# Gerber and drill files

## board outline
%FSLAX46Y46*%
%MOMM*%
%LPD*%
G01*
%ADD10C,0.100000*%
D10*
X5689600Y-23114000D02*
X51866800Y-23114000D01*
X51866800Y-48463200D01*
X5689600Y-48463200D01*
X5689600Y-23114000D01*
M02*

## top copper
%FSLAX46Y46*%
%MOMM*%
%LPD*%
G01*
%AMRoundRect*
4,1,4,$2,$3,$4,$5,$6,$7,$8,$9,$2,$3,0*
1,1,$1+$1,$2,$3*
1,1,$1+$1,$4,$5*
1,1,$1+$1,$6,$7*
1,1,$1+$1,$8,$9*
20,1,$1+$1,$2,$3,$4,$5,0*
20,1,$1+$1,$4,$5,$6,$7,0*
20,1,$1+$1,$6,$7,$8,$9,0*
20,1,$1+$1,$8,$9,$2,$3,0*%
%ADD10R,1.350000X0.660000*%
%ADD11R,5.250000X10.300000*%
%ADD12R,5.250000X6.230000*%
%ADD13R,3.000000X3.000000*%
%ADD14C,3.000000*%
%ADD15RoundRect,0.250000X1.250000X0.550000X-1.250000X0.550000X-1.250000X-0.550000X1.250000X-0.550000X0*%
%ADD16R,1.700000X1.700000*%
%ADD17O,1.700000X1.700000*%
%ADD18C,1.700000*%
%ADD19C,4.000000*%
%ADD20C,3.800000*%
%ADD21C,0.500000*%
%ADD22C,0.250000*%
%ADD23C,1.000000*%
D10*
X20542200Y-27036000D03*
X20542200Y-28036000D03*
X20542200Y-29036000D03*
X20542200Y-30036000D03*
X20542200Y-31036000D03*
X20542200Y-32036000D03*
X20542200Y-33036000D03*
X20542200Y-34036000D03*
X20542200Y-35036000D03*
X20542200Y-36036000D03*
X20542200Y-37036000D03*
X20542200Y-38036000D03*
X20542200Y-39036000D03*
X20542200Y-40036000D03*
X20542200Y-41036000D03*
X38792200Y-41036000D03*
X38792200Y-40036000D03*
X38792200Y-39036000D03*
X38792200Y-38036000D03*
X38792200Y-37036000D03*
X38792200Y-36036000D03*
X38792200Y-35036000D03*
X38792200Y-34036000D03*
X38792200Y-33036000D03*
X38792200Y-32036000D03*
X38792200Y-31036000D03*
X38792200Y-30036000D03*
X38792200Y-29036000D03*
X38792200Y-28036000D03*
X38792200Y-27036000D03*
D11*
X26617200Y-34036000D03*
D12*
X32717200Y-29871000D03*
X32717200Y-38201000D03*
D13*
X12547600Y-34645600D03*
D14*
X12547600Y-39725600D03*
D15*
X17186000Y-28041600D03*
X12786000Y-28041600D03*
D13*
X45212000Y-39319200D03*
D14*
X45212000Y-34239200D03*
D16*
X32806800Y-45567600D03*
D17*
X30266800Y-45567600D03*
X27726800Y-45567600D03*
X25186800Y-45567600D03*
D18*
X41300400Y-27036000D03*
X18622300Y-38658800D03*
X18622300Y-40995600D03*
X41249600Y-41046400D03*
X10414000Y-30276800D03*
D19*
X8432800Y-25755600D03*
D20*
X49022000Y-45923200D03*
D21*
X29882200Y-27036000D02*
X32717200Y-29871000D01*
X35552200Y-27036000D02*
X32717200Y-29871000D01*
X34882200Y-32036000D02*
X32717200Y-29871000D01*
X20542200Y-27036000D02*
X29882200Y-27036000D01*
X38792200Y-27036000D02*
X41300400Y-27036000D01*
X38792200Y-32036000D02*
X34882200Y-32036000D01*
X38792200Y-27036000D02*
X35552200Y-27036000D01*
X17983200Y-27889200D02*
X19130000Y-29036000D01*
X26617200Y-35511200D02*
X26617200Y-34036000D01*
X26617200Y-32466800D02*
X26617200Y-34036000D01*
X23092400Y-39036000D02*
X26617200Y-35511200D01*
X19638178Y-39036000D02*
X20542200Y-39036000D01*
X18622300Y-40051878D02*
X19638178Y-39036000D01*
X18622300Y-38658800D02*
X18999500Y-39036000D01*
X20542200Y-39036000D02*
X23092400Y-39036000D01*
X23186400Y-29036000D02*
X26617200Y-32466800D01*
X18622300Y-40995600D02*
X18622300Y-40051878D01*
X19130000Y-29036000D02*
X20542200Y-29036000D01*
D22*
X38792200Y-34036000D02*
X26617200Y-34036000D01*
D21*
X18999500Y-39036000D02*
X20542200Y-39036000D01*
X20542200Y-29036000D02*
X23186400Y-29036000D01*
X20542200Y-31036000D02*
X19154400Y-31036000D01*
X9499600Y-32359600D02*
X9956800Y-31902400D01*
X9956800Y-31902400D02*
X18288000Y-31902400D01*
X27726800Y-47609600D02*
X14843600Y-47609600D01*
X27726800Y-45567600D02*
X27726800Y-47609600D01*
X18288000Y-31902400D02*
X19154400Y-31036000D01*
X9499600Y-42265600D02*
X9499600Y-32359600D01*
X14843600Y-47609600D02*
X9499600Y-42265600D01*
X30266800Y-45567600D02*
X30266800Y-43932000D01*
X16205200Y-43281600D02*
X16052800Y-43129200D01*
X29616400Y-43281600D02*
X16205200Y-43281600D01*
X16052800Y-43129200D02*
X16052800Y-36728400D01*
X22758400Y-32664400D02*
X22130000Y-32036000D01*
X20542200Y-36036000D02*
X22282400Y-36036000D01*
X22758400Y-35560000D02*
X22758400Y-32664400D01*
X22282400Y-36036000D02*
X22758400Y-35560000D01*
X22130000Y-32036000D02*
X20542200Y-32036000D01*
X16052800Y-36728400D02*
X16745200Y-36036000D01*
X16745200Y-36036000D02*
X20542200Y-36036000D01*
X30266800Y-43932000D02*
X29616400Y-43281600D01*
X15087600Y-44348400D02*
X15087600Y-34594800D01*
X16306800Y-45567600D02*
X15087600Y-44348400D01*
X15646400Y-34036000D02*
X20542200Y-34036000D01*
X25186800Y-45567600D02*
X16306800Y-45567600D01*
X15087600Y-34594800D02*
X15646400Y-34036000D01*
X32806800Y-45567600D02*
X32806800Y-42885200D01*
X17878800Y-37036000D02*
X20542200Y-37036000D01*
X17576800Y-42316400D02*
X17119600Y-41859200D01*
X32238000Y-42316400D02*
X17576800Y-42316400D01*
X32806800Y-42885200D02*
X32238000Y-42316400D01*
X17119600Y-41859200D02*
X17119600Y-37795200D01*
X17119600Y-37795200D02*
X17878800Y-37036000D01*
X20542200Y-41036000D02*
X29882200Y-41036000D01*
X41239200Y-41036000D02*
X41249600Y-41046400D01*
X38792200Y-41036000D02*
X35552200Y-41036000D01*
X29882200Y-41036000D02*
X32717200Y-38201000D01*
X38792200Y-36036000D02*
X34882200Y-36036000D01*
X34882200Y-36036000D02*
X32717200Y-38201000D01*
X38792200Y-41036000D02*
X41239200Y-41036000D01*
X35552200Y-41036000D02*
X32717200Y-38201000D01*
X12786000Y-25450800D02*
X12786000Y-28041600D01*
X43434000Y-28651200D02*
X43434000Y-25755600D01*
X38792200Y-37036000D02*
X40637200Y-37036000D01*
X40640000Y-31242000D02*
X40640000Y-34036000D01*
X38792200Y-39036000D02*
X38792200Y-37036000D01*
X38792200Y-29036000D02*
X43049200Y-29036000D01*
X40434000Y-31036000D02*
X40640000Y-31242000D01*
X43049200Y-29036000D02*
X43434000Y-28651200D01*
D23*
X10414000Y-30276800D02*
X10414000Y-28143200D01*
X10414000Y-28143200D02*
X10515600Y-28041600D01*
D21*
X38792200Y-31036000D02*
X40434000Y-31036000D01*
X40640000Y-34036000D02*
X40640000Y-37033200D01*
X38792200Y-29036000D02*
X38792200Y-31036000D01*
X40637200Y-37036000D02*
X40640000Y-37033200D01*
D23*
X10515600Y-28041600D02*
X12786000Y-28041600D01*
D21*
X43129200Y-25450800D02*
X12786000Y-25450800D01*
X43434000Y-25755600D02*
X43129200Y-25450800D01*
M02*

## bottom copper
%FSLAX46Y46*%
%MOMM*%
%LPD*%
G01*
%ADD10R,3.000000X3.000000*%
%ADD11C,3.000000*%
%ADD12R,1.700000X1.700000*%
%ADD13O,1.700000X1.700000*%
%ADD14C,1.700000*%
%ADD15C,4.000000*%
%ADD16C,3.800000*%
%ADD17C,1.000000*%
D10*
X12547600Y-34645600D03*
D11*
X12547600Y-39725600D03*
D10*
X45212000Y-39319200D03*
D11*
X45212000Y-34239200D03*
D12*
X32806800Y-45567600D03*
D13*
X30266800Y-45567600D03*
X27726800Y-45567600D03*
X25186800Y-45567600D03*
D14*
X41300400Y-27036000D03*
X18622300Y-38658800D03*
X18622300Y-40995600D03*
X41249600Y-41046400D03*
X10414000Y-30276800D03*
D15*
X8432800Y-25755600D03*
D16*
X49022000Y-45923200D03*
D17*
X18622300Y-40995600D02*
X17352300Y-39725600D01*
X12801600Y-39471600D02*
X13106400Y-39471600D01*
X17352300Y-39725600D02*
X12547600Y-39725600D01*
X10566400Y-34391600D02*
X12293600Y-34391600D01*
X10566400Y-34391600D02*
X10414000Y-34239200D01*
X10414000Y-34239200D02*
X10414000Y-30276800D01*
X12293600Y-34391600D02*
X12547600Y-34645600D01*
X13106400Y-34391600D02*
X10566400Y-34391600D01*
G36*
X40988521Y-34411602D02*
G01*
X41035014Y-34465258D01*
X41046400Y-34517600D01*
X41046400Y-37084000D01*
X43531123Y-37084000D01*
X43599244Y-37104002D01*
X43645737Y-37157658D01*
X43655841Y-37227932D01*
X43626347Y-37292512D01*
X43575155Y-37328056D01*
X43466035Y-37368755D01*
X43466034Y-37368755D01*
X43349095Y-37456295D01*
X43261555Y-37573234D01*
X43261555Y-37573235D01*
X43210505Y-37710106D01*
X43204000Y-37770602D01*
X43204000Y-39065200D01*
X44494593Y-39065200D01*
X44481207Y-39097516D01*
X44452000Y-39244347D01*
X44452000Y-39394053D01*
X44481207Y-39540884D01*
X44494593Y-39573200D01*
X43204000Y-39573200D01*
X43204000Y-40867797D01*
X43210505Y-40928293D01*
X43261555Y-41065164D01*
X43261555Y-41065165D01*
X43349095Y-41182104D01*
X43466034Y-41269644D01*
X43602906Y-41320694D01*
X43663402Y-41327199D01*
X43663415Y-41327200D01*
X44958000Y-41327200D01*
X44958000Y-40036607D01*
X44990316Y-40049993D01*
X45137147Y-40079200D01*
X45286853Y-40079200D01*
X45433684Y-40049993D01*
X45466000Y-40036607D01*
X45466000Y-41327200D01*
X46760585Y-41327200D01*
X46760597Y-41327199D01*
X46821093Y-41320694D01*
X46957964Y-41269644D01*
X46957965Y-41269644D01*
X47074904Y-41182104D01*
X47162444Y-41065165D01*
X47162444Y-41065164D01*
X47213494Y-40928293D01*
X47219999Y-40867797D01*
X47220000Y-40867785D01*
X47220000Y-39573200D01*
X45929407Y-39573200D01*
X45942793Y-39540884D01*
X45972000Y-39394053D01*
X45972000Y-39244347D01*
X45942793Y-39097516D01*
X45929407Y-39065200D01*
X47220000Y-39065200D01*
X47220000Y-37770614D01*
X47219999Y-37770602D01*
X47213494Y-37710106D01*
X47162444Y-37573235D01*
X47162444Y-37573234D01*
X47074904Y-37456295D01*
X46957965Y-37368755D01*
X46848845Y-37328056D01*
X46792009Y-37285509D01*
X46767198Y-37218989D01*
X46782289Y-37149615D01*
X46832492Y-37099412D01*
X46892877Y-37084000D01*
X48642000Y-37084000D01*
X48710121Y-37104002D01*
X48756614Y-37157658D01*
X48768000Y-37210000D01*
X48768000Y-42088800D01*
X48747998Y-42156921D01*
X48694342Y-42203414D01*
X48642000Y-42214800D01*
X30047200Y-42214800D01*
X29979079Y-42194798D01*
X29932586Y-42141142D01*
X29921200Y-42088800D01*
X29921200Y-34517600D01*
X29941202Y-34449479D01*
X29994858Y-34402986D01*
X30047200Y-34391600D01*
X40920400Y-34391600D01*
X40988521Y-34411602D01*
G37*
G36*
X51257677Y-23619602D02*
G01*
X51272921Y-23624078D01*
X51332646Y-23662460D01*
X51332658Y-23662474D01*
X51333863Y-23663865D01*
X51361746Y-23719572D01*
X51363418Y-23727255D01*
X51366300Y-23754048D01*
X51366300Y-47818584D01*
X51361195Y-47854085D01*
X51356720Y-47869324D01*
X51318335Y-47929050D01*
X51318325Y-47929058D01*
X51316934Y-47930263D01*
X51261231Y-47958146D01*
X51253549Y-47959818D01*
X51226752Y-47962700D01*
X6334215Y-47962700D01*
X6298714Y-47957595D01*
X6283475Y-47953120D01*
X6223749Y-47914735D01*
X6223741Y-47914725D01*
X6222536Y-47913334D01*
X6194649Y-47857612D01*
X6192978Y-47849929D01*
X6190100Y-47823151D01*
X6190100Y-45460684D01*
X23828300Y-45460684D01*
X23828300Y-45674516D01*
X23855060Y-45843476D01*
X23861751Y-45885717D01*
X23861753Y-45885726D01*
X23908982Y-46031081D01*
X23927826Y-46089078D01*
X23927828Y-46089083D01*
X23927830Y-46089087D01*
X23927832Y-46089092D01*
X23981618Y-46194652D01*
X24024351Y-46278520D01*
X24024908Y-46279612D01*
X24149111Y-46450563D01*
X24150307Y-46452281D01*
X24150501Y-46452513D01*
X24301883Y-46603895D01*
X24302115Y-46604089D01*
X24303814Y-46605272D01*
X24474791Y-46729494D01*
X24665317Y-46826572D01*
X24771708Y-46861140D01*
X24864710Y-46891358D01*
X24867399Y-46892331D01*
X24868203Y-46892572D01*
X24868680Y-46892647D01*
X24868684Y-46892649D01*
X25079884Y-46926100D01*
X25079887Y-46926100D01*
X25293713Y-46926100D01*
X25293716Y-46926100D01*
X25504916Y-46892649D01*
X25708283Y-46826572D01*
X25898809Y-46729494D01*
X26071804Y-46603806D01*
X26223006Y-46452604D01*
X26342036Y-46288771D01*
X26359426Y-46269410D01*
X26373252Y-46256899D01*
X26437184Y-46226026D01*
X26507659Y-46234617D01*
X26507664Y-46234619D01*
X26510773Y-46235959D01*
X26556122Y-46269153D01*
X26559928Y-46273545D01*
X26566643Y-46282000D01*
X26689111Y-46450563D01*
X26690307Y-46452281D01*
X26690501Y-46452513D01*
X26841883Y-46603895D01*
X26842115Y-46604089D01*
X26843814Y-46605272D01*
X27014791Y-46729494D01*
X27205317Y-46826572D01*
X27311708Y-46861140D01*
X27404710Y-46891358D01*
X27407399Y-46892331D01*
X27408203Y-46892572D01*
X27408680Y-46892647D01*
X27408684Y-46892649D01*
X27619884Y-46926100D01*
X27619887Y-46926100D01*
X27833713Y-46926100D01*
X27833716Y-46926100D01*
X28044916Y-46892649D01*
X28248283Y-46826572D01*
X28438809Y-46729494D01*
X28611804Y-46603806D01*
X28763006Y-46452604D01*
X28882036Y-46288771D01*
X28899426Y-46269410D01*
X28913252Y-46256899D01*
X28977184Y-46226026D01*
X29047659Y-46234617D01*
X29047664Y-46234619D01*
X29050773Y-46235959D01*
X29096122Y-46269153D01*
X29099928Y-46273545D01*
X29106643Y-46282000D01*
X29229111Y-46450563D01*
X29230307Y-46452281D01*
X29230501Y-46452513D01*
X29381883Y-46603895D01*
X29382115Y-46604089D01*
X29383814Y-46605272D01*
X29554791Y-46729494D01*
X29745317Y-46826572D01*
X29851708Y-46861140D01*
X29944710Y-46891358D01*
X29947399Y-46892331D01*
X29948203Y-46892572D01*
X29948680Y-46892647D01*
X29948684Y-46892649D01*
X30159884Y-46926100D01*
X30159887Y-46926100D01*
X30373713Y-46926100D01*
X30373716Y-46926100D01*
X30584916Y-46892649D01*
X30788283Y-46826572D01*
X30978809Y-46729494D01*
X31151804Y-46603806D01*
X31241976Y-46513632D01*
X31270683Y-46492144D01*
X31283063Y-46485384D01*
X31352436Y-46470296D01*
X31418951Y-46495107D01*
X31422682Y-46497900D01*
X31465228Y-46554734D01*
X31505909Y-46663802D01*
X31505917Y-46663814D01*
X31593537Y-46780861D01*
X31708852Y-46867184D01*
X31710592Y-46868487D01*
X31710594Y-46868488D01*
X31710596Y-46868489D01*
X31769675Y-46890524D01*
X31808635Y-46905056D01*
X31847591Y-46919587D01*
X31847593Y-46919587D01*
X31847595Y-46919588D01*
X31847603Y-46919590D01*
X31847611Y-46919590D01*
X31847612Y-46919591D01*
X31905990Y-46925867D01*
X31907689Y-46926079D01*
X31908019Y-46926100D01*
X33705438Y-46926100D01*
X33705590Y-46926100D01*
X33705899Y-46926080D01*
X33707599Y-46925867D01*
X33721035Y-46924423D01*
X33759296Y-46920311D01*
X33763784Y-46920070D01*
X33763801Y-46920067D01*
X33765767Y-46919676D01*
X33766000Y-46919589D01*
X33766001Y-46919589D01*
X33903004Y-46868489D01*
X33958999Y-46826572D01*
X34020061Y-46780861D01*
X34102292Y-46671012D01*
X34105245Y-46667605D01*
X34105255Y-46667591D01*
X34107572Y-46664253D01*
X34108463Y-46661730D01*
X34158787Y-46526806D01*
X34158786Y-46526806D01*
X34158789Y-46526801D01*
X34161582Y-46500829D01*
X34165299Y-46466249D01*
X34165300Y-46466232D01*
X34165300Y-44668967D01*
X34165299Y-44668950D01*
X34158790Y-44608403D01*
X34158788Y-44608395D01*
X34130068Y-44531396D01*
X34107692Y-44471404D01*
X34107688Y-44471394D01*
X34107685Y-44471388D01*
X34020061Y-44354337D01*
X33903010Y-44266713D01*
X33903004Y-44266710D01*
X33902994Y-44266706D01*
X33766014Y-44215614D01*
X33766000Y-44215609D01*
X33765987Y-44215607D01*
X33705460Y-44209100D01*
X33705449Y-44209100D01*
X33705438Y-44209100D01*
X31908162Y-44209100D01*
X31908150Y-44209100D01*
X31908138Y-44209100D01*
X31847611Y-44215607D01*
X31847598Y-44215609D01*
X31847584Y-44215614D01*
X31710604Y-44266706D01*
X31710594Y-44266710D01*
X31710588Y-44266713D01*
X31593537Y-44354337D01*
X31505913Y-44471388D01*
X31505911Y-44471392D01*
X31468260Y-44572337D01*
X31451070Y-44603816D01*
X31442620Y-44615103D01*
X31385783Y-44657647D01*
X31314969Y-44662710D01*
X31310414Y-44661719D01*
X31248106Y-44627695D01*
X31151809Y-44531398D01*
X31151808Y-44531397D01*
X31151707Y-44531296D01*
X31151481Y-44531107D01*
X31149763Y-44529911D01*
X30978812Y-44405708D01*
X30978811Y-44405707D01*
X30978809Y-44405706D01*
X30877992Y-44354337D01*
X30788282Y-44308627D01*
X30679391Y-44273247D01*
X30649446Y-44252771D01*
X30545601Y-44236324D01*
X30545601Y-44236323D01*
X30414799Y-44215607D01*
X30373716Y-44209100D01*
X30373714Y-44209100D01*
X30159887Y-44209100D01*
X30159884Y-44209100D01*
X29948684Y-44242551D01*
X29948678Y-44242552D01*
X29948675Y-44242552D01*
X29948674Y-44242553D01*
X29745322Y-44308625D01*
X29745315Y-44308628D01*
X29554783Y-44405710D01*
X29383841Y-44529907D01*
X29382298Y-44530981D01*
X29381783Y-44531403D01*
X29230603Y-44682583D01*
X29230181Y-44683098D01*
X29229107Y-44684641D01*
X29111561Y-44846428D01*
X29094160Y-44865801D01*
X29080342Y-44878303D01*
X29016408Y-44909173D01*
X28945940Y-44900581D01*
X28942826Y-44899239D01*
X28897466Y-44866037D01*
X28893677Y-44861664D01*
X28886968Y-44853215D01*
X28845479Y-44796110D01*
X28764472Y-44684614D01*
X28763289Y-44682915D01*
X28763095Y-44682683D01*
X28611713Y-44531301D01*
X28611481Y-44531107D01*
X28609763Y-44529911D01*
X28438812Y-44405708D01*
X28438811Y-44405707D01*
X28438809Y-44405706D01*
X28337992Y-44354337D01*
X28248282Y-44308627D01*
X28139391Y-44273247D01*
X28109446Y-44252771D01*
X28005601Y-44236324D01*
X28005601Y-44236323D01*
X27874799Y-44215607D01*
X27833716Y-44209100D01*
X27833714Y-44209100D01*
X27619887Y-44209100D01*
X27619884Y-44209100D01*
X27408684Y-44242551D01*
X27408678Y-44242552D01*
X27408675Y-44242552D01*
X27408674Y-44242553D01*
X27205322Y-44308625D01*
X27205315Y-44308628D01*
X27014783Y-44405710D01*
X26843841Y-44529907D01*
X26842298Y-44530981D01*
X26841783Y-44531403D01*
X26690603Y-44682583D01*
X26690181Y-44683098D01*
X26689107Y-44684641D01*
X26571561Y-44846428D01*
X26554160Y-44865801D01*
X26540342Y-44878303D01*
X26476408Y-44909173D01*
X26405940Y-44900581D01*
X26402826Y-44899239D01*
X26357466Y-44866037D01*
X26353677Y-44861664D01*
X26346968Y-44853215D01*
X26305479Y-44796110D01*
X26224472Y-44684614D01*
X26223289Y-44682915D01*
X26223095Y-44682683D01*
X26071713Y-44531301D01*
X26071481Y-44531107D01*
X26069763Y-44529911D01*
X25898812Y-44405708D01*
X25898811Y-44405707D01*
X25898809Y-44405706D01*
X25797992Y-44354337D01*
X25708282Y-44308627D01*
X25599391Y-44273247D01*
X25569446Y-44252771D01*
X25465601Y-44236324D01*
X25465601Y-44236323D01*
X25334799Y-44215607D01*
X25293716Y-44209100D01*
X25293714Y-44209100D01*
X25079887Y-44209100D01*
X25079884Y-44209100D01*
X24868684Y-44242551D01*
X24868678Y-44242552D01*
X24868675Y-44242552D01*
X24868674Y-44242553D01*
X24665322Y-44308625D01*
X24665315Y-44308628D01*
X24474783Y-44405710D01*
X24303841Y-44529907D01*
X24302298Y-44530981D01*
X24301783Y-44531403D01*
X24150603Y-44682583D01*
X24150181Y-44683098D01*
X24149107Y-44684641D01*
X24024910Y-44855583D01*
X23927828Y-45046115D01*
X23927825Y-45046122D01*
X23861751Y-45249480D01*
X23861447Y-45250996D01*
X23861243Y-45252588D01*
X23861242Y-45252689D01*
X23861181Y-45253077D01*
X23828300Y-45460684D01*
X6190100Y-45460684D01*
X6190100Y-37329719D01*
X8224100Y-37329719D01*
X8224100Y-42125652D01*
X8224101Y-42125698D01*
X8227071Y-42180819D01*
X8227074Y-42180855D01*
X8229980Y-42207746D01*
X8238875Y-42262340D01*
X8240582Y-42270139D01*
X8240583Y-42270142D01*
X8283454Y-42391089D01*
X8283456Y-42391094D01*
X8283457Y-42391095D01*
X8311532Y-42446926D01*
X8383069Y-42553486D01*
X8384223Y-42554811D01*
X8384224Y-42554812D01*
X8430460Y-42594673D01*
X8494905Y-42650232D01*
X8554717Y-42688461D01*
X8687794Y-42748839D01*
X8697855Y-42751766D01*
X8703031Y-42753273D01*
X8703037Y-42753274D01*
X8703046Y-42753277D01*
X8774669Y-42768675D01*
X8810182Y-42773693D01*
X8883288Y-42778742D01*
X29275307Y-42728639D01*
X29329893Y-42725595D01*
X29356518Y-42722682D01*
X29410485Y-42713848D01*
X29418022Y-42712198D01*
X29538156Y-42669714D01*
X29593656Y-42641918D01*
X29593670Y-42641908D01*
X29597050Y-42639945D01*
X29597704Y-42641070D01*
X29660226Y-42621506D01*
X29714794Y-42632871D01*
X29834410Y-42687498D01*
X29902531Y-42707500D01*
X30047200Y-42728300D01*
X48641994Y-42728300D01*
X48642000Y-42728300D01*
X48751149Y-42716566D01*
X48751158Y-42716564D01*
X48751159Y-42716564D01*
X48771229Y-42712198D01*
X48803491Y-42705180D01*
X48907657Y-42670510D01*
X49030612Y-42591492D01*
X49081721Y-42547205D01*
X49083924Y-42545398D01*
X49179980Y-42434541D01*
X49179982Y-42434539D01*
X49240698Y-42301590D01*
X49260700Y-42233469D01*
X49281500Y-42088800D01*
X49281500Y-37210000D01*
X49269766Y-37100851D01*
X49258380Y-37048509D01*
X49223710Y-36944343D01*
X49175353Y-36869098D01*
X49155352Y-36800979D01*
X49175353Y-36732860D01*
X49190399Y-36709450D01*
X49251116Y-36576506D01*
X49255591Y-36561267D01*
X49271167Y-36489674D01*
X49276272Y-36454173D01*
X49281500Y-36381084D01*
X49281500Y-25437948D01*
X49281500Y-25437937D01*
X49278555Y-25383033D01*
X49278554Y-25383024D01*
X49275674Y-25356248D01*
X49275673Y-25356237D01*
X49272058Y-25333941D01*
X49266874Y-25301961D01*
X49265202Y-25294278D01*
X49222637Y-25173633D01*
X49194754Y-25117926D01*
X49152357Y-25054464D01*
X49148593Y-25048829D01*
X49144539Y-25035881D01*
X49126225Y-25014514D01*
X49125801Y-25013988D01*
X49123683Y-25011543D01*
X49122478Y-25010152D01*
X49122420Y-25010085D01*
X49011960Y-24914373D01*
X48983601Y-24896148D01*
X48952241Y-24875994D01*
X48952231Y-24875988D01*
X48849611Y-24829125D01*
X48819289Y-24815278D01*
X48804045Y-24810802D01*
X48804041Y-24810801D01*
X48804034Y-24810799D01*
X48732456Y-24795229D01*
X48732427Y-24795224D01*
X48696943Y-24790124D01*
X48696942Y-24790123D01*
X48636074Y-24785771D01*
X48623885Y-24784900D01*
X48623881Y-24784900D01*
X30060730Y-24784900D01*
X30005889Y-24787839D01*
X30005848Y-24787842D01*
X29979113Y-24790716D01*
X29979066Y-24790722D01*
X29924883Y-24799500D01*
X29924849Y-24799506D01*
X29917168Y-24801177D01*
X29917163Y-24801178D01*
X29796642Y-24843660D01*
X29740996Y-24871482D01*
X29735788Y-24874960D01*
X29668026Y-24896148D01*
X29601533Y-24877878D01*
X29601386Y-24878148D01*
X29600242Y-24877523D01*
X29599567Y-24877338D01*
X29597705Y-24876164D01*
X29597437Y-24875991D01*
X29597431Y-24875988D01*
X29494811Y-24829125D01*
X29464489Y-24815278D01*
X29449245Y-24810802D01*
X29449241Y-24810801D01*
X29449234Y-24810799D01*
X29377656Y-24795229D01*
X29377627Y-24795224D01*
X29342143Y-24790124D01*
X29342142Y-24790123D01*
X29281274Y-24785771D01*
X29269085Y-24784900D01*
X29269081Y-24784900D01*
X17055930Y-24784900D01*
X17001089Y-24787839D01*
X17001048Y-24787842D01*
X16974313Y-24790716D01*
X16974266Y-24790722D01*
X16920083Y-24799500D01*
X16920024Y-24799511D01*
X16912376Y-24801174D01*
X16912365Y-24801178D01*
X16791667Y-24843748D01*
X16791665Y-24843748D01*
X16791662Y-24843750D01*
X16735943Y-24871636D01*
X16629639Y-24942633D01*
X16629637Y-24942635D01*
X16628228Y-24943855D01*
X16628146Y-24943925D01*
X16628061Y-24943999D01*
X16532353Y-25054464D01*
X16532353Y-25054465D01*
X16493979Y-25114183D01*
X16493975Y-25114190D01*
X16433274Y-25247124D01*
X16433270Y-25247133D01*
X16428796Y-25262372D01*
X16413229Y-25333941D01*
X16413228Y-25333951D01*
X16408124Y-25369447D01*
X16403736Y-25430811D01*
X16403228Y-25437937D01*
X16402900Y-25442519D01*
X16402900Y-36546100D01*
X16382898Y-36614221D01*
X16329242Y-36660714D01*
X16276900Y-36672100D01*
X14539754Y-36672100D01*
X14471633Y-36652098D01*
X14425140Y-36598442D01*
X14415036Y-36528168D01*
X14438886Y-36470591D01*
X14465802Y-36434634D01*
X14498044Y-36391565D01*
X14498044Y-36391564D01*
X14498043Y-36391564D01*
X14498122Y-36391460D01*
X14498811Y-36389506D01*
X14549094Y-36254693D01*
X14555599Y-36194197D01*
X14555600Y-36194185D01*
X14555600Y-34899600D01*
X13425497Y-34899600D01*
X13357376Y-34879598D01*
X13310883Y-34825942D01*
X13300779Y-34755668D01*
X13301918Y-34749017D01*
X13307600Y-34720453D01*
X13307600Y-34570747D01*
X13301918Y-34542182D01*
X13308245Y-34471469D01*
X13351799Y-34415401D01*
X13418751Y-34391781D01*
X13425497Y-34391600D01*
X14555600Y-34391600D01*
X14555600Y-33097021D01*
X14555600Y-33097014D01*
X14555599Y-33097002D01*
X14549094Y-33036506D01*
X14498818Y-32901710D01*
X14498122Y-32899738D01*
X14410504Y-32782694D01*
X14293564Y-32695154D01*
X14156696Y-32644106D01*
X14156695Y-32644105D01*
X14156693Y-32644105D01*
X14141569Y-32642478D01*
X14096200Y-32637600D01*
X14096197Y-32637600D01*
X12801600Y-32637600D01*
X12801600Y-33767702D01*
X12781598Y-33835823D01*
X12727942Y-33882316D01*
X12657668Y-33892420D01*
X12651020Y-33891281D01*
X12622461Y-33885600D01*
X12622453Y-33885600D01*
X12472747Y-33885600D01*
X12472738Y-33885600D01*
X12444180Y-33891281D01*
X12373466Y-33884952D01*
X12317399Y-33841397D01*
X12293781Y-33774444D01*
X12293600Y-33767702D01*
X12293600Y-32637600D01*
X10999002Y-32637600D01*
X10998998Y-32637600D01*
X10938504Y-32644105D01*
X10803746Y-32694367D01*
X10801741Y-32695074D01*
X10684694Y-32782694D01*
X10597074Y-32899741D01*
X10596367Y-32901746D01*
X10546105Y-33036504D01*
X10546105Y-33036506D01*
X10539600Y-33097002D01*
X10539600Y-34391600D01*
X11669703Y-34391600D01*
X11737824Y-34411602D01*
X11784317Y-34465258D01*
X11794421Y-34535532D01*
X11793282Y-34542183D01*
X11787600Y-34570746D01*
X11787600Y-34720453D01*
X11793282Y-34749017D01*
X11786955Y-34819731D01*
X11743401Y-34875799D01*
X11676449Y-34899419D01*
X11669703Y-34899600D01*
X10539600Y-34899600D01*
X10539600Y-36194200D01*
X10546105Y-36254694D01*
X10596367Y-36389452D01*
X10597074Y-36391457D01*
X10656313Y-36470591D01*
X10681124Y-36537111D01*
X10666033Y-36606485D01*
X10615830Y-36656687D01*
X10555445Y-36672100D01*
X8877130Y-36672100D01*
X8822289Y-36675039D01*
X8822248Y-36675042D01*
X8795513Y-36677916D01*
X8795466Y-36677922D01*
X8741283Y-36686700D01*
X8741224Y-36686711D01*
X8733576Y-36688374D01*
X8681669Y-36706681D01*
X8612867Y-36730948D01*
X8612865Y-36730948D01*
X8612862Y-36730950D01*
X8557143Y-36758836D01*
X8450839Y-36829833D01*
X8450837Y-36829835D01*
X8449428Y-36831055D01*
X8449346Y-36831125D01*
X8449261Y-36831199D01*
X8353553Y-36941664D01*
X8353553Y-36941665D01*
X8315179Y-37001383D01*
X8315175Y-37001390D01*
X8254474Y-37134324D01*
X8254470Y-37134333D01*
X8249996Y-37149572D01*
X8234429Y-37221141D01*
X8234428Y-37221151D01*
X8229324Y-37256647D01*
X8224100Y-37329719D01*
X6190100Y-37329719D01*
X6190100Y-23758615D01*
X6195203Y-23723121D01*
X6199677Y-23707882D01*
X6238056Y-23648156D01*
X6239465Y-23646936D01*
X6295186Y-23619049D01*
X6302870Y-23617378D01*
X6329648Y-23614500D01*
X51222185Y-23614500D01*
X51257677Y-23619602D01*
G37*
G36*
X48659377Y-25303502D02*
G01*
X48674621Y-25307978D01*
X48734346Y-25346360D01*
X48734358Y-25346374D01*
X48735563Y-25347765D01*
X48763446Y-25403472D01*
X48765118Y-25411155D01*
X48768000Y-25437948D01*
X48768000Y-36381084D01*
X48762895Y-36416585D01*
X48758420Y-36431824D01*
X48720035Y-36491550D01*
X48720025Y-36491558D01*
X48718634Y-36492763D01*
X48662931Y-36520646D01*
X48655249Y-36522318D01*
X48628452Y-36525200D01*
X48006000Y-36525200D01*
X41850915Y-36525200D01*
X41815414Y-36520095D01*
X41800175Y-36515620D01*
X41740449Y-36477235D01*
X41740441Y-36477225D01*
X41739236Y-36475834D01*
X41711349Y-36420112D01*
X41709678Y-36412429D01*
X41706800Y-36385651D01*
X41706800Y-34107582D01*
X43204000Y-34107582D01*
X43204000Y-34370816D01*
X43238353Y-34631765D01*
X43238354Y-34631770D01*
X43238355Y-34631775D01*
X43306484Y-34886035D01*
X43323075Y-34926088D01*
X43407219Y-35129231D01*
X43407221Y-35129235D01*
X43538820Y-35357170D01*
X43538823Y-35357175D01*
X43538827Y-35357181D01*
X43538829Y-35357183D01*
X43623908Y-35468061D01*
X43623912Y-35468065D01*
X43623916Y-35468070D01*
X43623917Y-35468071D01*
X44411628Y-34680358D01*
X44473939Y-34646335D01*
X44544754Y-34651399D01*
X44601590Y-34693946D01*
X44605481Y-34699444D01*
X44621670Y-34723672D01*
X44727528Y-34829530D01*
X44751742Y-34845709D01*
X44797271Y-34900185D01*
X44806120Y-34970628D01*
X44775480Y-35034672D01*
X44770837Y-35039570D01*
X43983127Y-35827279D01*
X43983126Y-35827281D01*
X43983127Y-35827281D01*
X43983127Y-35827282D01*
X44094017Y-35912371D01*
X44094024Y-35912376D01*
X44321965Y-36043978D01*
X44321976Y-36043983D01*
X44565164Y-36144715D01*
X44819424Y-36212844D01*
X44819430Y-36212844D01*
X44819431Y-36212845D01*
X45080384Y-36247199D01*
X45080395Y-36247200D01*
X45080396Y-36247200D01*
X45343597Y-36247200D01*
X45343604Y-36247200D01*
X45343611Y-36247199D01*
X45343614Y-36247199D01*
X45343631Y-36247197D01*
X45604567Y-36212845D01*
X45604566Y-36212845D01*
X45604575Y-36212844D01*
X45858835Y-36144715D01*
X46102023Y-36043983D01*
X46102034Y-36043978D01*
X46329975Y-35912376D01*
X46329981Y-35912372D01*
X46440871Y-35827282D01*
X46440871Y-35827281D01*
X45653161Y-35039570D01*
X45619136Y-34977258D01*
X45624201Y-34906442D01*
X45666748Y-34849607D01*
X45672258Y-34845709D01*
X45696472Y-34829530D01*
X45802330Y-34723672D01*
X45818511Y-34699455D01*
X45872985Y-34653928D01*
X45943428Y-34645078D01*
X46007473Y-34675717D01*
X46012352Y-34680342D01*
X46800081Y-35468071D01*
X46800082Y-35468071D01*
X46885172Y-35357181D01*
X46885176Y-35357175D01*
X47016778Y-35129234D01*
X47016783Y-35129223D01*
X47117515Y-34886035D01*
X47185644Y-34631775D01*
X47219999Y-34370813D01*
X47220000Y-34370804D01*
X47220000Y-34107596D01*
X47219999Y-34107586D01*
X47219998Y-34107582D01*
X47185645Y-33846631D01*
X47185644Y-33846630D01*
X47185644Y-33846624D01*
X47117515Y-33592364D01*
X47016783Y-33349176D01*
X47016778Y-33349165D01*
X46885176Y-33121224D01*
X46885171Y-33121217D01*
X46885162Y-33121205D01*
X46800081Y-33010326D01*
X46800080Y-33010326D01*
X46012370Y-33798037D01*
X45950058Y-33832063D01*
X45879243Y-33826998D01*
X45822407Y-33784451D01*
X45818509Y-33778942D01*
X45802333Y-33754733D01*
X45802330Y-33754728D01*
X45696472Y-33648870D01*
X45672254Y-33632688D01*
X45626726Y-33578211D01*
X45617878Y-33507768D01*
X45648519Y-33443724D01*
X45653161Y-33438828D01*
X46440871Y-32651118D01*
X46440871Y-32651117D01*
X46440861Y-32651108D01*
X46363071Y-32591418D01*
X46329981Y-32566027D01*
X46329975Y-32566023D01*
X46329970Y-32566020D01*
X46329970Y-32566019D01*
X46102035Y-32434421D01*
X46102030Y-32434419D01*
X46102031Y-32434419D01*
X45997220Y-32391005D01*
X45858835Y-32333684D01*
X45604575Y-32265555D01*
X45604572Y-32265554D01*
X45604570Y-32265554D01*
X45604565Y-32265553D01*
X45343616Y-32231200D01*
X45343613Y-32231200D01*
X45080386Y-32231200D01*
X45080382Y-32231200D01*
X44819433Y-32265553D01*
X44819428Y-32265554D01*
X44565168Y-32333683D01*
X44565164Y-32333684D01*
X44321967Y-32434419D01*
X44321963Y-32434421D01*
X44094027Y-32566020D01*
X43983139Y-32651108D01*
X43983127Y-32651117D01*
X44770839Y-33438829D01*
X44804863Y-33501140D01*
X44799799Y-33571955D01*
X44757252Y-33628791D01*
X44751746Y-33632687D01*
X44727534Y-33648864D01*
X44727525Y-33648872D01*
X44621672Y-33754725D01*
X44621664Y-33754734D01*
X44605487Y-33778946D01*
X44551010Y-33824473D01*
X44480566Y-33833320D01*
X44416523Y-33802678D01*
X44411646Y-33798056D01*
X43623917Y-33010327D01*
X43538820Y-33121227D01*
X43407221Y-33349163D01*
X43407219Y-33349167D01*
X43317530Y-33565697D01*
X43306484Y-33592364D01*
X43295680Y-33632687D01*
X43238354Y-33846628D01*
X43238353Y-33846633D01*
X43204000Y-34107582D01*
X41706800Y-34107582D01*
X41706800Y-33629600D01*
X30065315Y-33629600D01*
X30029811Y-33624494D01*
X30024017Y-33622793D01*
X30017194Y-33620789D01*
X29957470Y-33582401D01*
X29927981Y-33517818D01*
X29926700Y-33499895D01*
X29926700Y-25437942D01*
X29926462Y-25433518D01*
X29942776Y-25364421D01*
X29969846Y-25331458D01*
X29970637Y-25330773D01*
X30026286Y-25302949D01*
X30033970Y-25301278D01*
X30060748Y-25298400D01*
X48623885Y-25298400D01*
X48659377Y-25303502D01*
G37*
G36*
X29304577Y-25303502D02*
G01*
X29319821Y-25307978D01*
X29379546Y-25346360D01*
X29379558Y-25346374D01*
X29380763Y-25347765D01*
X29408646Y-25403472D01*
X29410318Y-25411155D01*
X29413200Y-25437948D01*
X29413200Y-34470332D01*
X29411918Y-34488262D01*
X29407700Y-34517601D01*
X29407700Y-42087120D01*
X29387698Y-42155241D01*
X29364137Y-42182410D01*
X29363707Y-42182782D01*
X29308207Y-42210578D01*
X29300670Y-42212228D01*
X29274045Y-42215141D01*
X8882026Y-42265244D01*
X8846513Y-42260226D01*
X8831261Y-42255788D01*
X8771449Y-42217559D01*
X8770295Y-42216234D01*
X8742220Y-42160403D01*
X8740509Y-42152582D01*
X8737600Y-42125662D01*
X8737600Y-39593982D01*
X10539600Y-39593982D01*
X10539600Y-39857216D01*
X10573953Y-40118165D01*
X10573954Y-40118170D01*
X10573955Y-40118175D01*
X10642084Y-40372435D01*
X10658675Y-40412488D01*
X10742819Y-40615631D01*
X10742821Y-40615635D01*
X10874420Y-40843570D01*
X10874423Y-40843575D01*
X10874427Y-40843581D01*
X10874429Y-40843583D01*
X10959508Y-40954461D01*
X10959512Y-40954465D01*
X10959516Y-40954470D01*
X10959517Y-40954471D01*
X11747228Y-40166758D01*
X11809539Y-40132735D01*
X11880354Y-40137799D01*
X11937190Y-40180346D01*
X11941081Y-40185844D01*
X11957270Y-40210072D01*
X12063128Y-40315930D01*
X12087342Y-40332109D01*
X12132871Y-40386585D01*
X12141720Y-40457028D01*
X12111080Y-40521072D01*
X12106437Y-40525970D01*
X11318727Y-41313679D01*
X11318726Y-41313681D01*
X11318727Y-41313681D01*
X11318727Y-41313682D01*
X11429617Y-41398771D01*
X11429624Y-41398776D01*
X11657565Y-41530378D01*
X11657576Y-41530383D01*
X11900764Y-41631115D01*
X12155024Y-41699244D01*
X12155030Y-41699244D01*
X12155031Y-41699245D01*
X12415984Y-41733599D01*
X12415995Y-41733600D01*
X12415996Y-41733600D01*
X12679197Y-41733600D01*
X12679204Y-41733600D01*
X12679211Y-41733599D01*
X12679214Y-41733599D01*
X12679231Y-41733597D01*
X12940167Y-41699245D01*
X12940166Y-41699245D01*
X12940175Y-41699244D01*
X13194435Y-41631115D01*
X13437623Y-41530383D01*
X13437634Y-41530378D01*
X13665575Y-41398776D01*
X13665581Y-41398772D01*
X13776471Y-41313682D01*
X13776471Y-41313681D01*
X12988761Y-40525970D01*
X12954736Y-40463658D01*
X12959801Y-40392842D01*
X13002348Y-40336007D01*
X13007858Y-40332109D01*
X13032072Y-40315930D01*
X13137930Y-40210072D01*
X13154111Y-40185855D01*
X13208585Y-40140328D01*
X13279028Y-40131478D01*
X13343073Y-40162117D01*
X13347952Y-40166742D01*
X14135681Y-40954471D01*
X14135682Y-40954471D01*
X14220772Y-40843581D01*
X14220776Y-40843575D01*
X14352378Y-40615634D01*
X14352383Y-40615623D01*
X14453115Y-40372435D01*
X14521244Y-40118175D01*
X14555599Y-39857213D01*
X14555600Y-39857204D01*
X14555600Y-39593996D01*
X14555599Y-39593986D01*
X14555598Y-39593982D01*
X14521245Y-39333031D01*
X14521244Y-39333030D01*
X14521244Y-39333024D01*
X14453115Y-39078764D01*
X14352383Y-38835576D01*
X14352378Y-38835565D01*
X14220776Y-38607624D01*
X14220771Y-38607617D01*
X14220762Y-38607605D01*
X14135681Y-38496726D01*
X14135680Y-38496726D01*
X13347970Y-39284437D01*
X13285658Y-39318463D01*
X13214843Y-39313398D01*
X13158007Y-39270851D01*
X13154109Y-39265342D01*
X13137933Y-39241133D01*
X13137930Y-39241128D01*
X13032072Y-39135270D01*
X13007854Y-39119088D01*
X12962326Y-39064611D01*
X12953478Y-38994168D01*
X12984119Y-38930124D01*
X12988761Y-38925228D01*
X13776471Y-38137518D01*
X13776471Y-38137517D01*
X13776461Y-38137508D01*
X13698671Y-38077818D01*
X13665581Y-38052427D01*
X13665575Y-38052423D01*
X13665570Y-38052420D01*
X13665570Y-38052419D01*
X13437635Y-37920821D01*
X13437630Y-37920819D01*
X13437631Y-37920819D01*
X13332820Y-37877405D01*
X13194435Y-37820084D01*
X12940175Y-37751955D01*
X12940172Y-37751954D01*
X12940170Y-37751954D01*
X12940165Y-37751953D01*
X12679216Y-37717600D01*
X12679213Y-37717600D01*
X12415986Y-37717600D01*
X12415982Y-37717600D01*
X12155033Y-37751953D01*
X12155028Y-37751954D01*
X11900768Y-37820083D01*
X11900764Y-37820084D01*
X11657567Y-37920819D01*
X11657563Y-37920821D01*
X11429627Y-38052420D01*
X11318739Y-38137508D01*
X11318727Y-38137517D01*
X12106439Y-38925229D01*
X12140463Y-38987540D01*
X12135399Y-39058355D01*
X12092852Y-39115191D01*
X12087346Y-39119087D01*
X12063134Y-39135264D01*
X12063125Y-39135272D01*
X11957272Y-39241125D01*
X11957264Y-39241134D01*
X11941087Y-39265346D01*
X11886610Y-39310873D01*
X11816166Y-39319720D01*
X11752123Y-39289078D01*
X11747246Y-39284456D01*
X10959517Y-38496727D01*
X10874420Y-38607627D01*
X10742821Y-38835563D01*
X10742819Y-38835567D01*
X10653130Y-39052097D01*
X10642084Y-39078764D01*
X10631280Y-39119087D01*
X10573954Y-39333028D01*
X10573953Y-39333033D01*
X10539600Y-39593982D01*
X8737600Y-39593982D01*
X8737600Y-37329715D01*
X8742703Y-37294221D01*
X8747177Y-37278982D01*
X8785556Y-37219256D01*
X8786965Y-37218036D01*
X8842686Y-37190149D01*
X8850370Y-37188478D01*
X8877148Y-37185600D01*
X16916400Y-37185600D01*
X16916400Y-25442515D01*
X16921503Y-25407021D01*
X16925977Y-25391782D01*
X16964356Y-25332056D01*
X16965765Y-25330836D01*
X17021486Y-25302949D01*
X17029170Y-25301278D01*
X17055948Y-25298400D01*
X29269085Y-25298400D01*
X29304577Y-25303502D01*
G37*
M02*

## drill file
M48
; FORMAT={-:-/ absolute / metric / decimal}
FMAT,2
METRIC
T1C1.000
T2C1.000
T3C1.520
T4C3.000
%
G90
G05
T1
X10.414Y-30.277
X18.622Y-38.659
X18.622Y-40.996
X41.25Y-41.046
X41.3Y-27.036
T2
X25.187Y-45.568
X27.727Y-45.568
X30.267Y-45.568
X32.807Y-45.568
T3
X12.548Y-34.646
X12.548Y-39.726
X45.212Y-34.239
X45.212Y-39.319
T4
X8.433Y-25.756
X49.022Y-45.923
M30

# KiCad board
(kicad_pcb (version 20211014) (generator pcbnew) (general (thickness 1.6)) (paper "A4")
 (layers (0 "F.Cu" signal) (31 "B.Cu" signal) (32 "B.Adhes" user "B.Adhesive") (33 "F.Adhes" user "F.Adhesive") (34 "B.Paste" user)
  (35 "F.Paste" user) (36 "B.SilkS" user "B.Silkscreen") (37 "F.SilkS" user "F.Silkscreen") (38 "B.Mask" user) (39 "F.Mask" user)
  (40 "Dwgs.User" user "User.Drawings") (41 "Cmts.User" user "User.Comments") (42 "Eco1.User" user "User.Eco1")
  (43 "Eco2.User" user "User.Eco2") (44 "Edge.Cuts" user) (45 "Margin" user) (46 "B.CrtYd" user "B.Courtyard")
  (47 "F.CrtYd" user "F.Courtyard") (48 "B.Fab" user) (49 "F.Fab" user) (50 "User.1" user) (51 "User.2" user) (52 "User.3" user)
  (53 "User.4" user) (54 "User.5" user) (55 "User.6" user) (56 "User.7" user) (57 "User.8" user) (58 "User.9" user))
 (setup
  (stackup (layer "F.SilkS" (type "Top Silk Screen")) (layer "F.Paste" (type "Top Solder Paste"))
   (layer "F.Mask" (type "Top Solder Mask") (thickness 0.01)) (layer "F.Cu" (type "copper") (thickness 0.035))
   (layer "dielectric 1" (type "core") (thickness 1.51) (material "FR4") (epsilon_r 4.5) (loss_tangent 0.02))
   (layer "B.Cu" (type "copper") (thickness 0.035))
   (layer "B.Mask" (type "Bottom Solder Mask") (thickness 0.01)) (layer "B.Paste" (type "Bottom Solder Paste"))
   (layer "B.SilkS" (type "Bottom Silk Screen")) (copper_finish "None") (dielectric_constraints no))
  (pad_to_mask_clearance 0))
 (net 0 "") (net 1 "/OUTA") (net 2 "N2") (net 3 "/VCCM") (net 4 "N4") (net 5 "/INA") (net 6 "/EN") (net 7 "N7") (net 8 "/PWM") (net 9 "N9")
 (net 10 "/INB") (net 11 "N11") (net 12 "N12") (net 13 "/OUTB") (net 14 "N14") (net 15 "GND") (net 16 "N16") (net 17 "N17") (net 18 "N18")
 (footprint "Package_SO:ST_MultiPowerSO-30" (layer "F.Cu") (at 29.6672 34.036)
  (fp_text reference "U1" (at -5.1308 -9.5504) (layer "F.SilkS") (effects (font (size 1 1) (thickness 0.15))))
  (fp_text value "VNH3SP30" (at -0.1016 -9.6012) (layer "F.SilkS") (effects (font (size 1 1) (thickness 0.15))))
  (pad "1" smd rect (at -9.125 -7 270) (size 0.66 1.35) (layers "F.Cu" "F.Paste" "F.Mask") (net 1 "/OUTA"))
  (pad "2" smd rect (at -9.125 -6 270) (size 0.66 1.35) (layers "F.Cu" "F.Paste" "F.Mask") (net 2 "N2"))
  (pad "3" smd rect (at -9.125 -5 270) (size 0.66 1.35) (layers "F.Cu" "F.Paste" "F.Mask") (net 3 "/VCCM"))
  (pad "4" smd rect (at -9.125 -4 270) (size 0.66 1.35) (layers "F.Cu" "F.Paste" "F.Mask") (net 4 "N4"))
  (pad "5" smd rect (at -9.125 -3 270) (size 0.66 1.35) (layers "F.Cu" "F.Paste" "F.Mask") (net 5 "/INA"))
  (pad "6" smd rect (at -9.125 -2 270) (size 0.66 1.35) (layers "F.Cu" "F.Paste" "F.Mask") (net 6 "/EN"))
  (pad "7" smd rect (at -9.125 -1 270) (size 0.66 1.35) (layers "F.Cu" "F.Paste" "F.Mask") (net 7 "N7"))
  (pad "8" smd rect (at -9.125 0 270) (size 0.66 1.35) (layers "F.Cu" "F.Paste" "F.Mask") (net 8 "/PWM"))
  (pad "9" smd rect (at -9.125 1 270) (size 0.66 1.35) (layers "F.Cu" "F.Paste" "F.Mask") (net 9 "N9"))
  (pad "10" smd rect (at -9.125 2 270) (size 0.66 1.35) (layers "F.Cu" "F.Paste" "F.Mask") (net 6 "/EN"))
  (pad "11" smd rect (at -9.125 3 270) (size 0.66 1.35) (layers "F.Cu" "F.Paste" "F.Mask") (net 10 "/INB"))
  (pad "12" smd rect (at -9.125 4 270) (size 0.66 1.35) (layers "F.Cu" "F.Paste" "F.Mask") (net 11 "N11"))
  (pad "13" smd rect (at -9.125 5 270) (size 0.66 1.35) (layers "F.Cu" "F.Paste" "F.Mask") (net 3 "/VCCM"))
  (pad "14" smd rect (at -9.125 6 270) (size 0.66 1.35) (layers "F.Cu" "F.Paste" "F.Mask") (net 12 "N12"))
  (pad "15" smd rect (at -9.125 7 270) (size 0.66 1.35) (layers "F.Cu" "F.Paste" "F.Mask") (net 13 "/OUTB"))
  (pad "16" smd rect (at 9.125 7 270) (size 0.66 1.35) (layers "F.Cu" "F.Paste" "F.Mask") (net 13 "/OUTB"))
  (pad "17" smd rect (at 9.125 6 270) (size 0.66 1.35) (layers "F.Cu" "F.Paste" "F.Mask") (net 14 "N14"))
  (pad "18" smd rect (at 9.125 5 270) (size 0.66 1.35) (layers "F.Cu" "F.Paste" "F.Mask") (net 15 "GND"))
  (pad "19" smd rect (at 9.125 4 270) (size 0.66 1.35) (layers "F.Cu" "F.Paste" "F.Mask") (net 15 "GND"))
  (pad "20" smd rect (at 9.125 3 270) (size 0.66 1.35) (layers "F.Cu" "F.Paste" "F.Mask") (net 15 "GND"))
  (pad "21" smd rect (at 9.125 2 270) (size 0.66 1.35) (layers "F.Cu" "F.Paste" "F.Mask") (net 13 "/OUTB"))
  (pad "22" smd rect (at 9.125 1 270) (size 0.66 1.35) (layers "F.Cu" "F.Paste" "F.Mask") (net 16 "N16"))
  (pad "23" smd rect (at 9.125 0 270) (size 0.66 1.35) (layers "F.Cu" "F.Paste" "F.Mask") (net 3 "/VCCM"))
  (pad "24" smd rect (at 9.125 -1 270) (size 0.66 1.35) (layers "F.Cu" "F.Paste" "F.Mask") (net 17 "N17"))
  (pad "25" smd rect (at 9.125 -2 270) (size 0.66 1.35) (layers "F.Cu" "F.Paste" "F.Mask") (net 1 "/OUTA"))
  (pad "26" smd rect (at 9.125 -3 270) (size 0.66 1.35) (layers "F.Cu" "F.Paste" "F.Mask") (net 15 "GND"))
  (pad "27" smd rect (at 9.125 -4 270) (size 0.66 1.35) (layers "F.Cu" "F.Paste" "F.Mask") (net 15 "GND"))
  (pad "28" smd rect (at 9.125 -5 270) (size 0.66 1.35) (layers "F.Cu" "F.Paste" "F.Mask") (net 15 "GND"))
  (pad "29" smd rect (at 9.125 -6 270) (size 0.66 1.35) (layers "F.Cu" "F.Paste" "F.Mask") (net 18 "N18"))
  (pad "30" smd rect (at 9.125 -7 270) (size 0.66 1.35) (layers "F.Cu" "F.Paste" "F.Mask") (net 1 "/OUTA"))
  (pad "31" smd rect (at -3.05 0) (size 5.25 10.3) (layers "F.Cu" "F.Paste" "F.Mask") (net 3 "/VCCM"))
  (pad "32" smd rect (at 3.05 -4.165) (size 5.25 6.23) (layers "F.Cu" "F.Paste" "F.Mask") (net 1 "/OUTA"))
  (pad "33" smd rect (at 3.05 4.165) (size 5.25 6.23) (layers "F.Cu" "F.Paste" "F.Mask") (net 13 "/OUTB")))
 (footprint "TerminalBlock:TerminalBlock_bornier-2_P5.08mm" (layer "F.Cu") (at 12.5476 34.6456 -90)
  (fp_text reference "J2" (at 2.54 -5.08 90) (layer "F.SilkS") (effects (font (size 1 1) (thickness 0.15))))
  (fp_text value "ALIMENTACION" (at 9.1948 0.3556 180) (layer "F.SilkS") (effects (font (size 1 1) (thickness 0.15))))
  (pad "1" thru_hole rect (at 0 0 270) (size 3 3) (drill 1.52) (layers *.Cu *.Mask) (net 15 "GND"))
  (pad "2" thru_hole circle (at 5.08 0 270) (size 3 3) (drill 1.52) (layers *.Cu *.Mask) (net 3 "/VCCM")))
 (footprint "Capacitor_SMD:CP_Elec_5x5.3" (layer "F.Cu") (at 14.986 28.0416 180)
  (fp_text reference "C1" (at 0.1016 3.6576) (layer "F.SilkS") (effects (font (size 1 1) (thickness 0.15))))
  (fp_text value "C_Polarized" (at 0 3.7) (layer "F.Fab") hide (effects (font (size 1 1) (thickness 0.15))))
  (pad "1" smd roundrect (at -2.2 0 180) (size 3 1.6) (layers "F.Cu" "F.Paste" "F.Mask") (roundrect_rratio 0.15625) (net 3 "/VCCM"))
  (pad "2" smd roundrect (at 2.2 0 180) (size 3 1.6) (layers "F.Cu" "F.Paste" "F.Mask") (roundrect_rratio 0.15625) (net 15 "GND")))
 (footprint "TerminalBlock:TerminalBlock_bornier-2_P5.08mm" (layer "F.Cu") (at 45.212 39.3192 90)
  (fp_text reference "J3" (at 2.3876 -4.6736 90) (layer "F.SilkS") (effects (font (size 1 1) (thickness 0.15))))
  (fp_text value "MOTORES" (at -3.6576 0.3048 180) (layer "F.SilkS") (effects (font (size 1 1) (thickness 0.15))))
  (pad "1" thru_hole rect (at 0 0 90) (size 3 3) (drill 1.52) (layers *.Cu *.Mask) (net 13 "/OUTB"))
  (pad "2" thru_hole circle (at 5.08 0 90) (size 3 3) (drill 1.52) (layers *.Cu *.Mask) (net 1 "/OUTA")))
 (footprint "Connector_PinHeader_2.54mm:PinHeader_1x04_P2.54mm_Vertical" (layer "F.Cu") (at 32.8068 45.5676 -90)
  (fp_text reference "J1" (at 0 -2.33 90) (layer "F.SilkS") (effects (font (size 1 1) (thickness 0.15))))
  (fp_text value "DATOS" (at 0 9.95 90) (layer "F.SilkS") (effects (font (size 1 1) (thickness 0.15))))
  (pad "1" thru_hole rect (at 0 0 270) (size 1.7 1.7) (drill 1) (layers *.Cu *.Mask) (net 10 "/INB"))
  (pad "2" thru_hole oval (at 0 2.54 270) (size 1.7 1.7) (drill 1) (layers *.Cu *.Mask) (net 6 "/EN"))
  (pad "3" thru_hole oval (at 0 5.08 270) (size 1.7 1.7) (drill 1) (layers *.Cu *.Mask) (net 5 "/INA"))
  (pad "4" thru_hole oval (at 0 7.62 270) (size 1.7 1.7) (drill 1) (layers *.Cu *.Mask) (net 8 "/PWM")))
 (gr_rect (start 5.6896 23.114) (end 51.8668 48.4632) (layer "Edge.Cuts") (width 0.1) (fill none))
 (segment (start 29.8822 27.036) (end 32.7172 29.871) (width 0.5) (layer "F.Cu") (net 1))
 (segment (start 35.5522 27.036) (end 32.7172 29.871) (width 0.5) (layer "F.Cu") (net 1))
 (segment (start 34.8822 32.036) (end 32.7172 29.871) (width 0.5) (layer "F.Cu") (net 1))
 (segment (start 20.5422 27.036) (end 29.8822 27.036) (width 0.5) (layer "F.Cu") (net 1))
 (segment (start 38.7922 27.036) (end 41.3004 27.036) (width 0.5) (layer "F.Cu") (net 1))
 (segment (start 38.7922 32.036) (end 34.8822 32.036) (width 0.5) (layer "F.Cu") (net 1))
 (segment (start 38.7922 27.036) (end 35.5522 27.036) (width 0.5) (layer "F.Cu") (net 1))
 (via (at 41.3004 27.036) (size 1.7) (drill 1) (layers "F.Cu" "B.Cu") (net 1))
 (segment (start 17.9832 27.8892) (end 19.13 29.036) (width 0.5) (layer "F.Cu") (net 3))
 (segment (start 26.6172 35.5112) (end 26.6172 34.036) (width 0.5) (layer "F.Cu") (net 3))
 (segment (start 26.6172 32.4668) (end 26.6172 34.036) (width 0.5) (layer "F.Cu") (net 3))
 (segment (start 23.0924 39.036) (end 26.6172 35.5112) (width 0.5) (layer "F.Cu") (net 3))
 (segment (start 19.638178 39.036) (end 20.5422 39.036) (width 0.5) (layer "F.Cu") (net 3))
 (segment (start 18.6223 40.051878) (end 19.638178 39.036) (width 0.5) (layer "F.Cu") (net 3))
 (segment (start 18.6223 38.6588) (end 18.9995 39.036) (width 0.5) (layer "F.Cu") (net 3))
 (segment (start 20.5422 39.036) (end 23.0924 39.036) (width 0.5) (layer "F.Cu") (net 3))
 (segment (start 23.1864 29.036) (end 26.6172 32.4668) (width 0.5) (layer "F.Cu") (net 3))
 (segment (start 18.6223 40.9956) (end 18.6223 40.051878) (width 0.5) (layer "F.Cu") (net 3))
 (segment (start 19.13 29.036) (end 20.5422 29.036) (width 0.5) (layer "F.Cu") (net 3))
 (segment (start 38.7922 34.036) (end 26.6172 34.036) (width 0.25) (layer "F.Cu") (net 3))
 (segment (start 18.9995 39.036) (end 20.5422 39.036) (width 0.5) (layer "F.Cu") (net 3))
 (segment (start 20.5422 29.036) (end 23.1864 29.036) (width 0.5) (layer "F.Cu") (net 3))
 (via (at 18.6223 38.6588) (size 1.7) (drill 1) (layers "F.Cu" "B.Cu") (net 3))
 (via (at 18.6223 40.9956) (size 1.7) (drill 1) (layers "F.Cu" "B.Cu") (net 3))
 (segment (start 18.6223 40.9956) (end 17.3523 39.7256) (width 1) (layer "B.Cu") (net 3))
 (segment (start 12.8016 39.4716) (end 13.1064 39.4716) (width 1) (layer "B.Cu") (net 3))
 (segment (start 17.3523 39.7256) (end 12.5476 39.7256) (width 1) (layer "B.Cu") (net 3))
 (segment (start 20.5422 31.036) (end 19.1544 31.036) (width 0.5) (layer "F.Cu") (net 5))
 (segment (start 9.4996 32.3596) (end 9.9568 31.9024) (width 0.5) (layer "F.Cu") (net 5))
 (segment (start 9.9568 31.9024) (end 18.288 31.9024) (width 0.5) (layer "F.Cu") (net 5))
 (segment (start 27.7268 47.6096) (end 14.8436 47.6096) (width 0.5) (layer "F.Cu") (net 5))
 (segment (start 27.7268 45.5676) (end 27.7268 47.6096) (width 0.5) (layer "F.Cu") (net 5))
 (segment (start 18.288 31.9024) (end 19.1544 31.036) (width 0.5) (layer "F.Cu") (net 5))
 (segment (start 9.4996 42.2656) (end 9.4996 32.3596) (width 0.5) (layer "F.Cu") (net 5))
 (segment (start 14.8436 47.6096) (end 9.4996 42.2656) (width 0.5) (layer "F.Cu") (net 5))
 (segment (start 30.2668 45.5676) (end 30.2668 43.932) (width 0.5) (layer "F.Cu") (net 6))
 (segment (start 16.2052 43.2816) (end 16.0528 43.1292) (width 0.5) (layer "F.Cu") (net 6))
 (segment (start 29.6164 43.2816) (end 16.2052 43.2816) (width 0.5) (layer "F.Cu") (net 6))
 (segment (start 16.0528 43.1292) (end 16.0528 36.7284) (width 0.5) (layer "F.Cu") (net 6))
 (segment (start 22.7584 32.6644) (end 22.13 32.036) (width 0.5) (layer "F.Cu") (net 6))
 (segment (start 20.5422 36.036) (end 22.2824 36.036) (width 0.5) (layer "F.Cu") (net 6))
 (segment (start 22.7584 35.56) (end 22.7584 32.6644) (width 0.5) (layer "F.Cu") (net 6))
 (segment (start 22.2824 36.036) (end 22.7584 35.56) (width 0.5) (layer "F.Cu") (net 6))
 (segment (start 22.13 32.036) (end 20.5422 32.036) (width 0.5) (layer "F.Cu") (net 6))
 (segment (start 16.0528 36.7284) (end 16.7452 36.036) (width 0.5) (layer "F.Cu") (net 6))
 (segment (start 16.7452 36.036) (end 20.5422 36.036) (width 0.5) (layer "F.Cu") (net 6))
 (segment (start 30.2668 43.932) (end 29.6164 43.2816) (width 0.5) (layer "F.Cu") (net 6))
 (segment (start 15.0876 44.3484) (end 15.0876 34.5948) (width 0.5) (layer "F.Cu") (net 8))
 (segment (start 16.3068 45.5676) (end 15.0876 44.3484) (width 0.5) (layer "F.Cu") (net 8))
 (segment (start 15.6464 34.036) (end 20.5422 34.036) (width 0.5) (layer "F.Cu") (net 8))
 (segment (start 25.1868 45.5676) (end 16.3068 45.5676) (width 0.5) (layer "F.Cu") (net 8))
 (segment (start 15.0876 34.5948) (end 15.6464 34.036) (width 0.5) (layer "F.Cu") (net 8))
 (segment (start 32.8068 45.5676) (end 32.8068 42.8852) (width 0.5) (layer "F.Cu") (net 10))
 (segment (start 17.8788 37.036) (end 20.5422 37.036) (width 0.5) (layer "F.Cu") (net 10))
 (segment (start 17.5768 42.3164) (end 17.1196 41.8592) (width 0.5) (layer "F.Cu") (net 10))
 (segment (start 32.238 42.3164) (end 17.5768 42.3164) (width 0.5) (layer "F.Cu") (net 10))
 (segment (start 32.8068 42.8852) (end 32.238 42.3164) (width 0.5) (layer "F.Cu") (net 10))
 (segment (start 17.1196 41.8592) (end 17.1196 37.7952) (width 0.5) (layer "F.Cu") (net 10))
 (segment (start 17.1196 37.7952) (end 17.8788 37.036) (width 0.5) (layer "F.Cu") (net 10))
 (segment (start 20.5422 41.036) (end 29.8822 41.036) (width 0.5) (layer "F.Cu") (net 13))
 (segment (start 41.2392 41.036) (end 41.2496 41.0464) (width 0.5) (layer "F.Cu") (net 13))
 (segment (start 38.7922 41.036) (end 35.5522 41.036) (width 0.5) (layer "F.Cu") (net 13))
 (segment (start 29.8822 41.036) (end 32.7172 38.201) (width 0.5) (layer "F.Cu") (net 13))
 (segment (start 38.7922 36.036) (end 34.8822 36.036) (width 0.5) (layer "F.Cu") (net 13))
 (segment (start 34.8822 36.036) (end 32.7172 38.201) (width 0.5) (layer "F.Cu") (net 13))
 (segment (start 38.7922 41.036) (end 41.2392 41.036) (width 0.5) (layer "F.Cu") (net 13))
 (segment (start 35.5522 41.036) (end 32.7172 38.201) (width 0.5) (layer "F.Cu") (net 13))
 (via (at 41.2496 41.0464) (size 1.7) (drill 1) (layers "F.Cu" "B.Cu") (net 13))
 (segment (start 12.786 25.4508) (end 12.786 28.0416) (width 0.5) (layer "F.Cu") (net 15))
 (segment (start 43.434 28.6512) (end 43.434 25.7556) (width 0.5) (layer "F.Cu") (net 15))
 (segment (start 38.7922 37.036) (end 40.6372 37.036) (width 0.5) (layer "F.Cu") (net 15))
 (segment (start 40.64 31.242) (end 40.64 34.036) (width 0.5) (layer "F.Cu") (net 15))
 (segment (start 38.7922 39.036) (end 38.7922 37.036) (width 0.5) (layer "F.Cu") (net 15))
 (segment (start 38.7922 29.036) (end 43.0492 29.036) (width 0.5) (layer "F.Cu") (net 15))
 (segment (start 40.434 31.036) (end 40.64 31.242) (width 0.5) (layer "F.Cu") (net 15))
 (segment (start 43.0492 29.036) (end 43.434 28.6512) (width 0.5) (layer "F.Cu") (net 15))
 (segment (start 10.414 30.2768) (end 10.414 28.1432) (width 1) (layer "F.Cu") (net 15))
 (segment (start 10.414 28.1432) (end 10.5156 28.0416) (width 1) (layer "F.Cu") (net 15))
 (segment (start 38.7922 31.036) (end 40.434 31.036) (width 0.5) (layer "F.Cu") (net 15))
 (segment (start 40.64 34.036) (end 40.64 37.0332) (width 0.5) (layer "F.Cu") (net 15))
 (segment (start 38.7922 29.036) (end 38.7922 31.036) (width 0.5) (layer "F.Cu") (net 15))
 (segment (start 40.6372 37.036) (end 40.64 37.0332) (width 0.5) (layer "F.Cu") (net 15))
 (segment (start 10.5156 28.0416) (end 12.786 28.0416) (width 1) (layer "F.Cu") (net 15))
 (segment (start 43.1292 25.4508) (end 12.786 25.4508) (width 0.5) (layer "F.Cu") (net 15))
 (segment (start 43.434 25.7556) (end 43.1292 25.4508) (width 0.5) (layer "F.Cu") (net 15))
 (via (at 10.414 30.2768) (size 1.7) (drill 1) (layers "F.Cu" "B.Cu") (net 15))
 (via (at 8.4328 25.7556) (size 4) (drill 3) (layers "F.Cu" "B.Cu") (free) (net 15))
 (via (at 49.022 45.9232) (size 3.8) (drill 3) (layers "F.Cu" "B.Cu") (free) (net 15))
 (segment (start 10.5664 34.3916) (end 12.2936 34.3916) (width 1) (layer "B.Cu") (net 15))
 (segment (start 10.5664 34.3916) (end 10.414 34.2392) (width 1) (layer "B.Cu") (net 15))
 (segment (start 10.414 34.2392) (end 10.414 30.2768) (width 1) (layer "B.Cu") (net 15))
 (segment (start 12.2936 34.3916) (end 12.5476 34.6456) (width 1) (layer "B.Cu") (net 15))
 (segment (start 13.1064 34.3916) (end 10.5664 34.3916) (width 1) (layer "B.Cu") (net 15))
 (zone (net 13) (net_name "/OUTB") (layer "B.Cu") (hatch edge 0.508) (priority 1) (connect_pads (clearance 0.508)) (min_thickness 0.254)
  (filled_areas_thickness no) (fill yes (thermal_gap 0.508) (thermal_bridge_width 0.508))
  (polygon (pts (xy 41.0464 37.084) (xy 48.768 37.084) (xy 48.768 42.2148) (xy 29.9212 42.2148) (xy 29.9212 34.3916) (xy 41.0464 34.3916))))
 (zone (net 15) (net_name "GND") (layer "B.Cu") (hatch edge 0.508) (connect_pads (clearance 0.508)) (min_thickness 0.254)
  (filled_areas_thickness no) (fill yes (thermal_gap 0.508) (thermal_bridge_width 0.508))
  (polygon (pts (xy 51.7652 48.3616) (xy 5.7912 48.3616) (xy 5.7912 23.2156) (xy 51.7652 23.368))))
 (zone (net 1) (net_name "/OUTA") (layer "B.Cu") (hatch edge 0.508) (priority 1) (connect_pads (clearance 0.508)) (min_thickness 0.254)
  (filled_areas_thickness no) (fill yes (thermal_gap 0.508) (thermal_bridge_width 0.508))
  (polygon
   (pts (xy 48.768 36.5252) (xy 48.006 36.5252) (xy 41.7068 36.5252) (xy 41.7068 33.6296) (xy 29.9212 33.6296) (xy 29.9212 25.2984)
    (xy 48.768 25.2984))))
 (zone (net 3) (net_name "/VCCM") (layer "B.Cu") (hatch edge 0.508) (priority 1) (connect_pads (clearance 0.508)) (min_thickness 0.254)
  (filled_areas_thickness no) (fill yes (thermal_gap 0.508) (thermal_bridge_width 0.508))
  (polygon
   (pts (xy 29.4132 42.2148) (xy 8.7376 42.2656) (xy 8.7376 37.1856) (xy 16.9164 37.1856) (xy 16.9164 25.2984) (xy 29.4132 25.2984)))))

